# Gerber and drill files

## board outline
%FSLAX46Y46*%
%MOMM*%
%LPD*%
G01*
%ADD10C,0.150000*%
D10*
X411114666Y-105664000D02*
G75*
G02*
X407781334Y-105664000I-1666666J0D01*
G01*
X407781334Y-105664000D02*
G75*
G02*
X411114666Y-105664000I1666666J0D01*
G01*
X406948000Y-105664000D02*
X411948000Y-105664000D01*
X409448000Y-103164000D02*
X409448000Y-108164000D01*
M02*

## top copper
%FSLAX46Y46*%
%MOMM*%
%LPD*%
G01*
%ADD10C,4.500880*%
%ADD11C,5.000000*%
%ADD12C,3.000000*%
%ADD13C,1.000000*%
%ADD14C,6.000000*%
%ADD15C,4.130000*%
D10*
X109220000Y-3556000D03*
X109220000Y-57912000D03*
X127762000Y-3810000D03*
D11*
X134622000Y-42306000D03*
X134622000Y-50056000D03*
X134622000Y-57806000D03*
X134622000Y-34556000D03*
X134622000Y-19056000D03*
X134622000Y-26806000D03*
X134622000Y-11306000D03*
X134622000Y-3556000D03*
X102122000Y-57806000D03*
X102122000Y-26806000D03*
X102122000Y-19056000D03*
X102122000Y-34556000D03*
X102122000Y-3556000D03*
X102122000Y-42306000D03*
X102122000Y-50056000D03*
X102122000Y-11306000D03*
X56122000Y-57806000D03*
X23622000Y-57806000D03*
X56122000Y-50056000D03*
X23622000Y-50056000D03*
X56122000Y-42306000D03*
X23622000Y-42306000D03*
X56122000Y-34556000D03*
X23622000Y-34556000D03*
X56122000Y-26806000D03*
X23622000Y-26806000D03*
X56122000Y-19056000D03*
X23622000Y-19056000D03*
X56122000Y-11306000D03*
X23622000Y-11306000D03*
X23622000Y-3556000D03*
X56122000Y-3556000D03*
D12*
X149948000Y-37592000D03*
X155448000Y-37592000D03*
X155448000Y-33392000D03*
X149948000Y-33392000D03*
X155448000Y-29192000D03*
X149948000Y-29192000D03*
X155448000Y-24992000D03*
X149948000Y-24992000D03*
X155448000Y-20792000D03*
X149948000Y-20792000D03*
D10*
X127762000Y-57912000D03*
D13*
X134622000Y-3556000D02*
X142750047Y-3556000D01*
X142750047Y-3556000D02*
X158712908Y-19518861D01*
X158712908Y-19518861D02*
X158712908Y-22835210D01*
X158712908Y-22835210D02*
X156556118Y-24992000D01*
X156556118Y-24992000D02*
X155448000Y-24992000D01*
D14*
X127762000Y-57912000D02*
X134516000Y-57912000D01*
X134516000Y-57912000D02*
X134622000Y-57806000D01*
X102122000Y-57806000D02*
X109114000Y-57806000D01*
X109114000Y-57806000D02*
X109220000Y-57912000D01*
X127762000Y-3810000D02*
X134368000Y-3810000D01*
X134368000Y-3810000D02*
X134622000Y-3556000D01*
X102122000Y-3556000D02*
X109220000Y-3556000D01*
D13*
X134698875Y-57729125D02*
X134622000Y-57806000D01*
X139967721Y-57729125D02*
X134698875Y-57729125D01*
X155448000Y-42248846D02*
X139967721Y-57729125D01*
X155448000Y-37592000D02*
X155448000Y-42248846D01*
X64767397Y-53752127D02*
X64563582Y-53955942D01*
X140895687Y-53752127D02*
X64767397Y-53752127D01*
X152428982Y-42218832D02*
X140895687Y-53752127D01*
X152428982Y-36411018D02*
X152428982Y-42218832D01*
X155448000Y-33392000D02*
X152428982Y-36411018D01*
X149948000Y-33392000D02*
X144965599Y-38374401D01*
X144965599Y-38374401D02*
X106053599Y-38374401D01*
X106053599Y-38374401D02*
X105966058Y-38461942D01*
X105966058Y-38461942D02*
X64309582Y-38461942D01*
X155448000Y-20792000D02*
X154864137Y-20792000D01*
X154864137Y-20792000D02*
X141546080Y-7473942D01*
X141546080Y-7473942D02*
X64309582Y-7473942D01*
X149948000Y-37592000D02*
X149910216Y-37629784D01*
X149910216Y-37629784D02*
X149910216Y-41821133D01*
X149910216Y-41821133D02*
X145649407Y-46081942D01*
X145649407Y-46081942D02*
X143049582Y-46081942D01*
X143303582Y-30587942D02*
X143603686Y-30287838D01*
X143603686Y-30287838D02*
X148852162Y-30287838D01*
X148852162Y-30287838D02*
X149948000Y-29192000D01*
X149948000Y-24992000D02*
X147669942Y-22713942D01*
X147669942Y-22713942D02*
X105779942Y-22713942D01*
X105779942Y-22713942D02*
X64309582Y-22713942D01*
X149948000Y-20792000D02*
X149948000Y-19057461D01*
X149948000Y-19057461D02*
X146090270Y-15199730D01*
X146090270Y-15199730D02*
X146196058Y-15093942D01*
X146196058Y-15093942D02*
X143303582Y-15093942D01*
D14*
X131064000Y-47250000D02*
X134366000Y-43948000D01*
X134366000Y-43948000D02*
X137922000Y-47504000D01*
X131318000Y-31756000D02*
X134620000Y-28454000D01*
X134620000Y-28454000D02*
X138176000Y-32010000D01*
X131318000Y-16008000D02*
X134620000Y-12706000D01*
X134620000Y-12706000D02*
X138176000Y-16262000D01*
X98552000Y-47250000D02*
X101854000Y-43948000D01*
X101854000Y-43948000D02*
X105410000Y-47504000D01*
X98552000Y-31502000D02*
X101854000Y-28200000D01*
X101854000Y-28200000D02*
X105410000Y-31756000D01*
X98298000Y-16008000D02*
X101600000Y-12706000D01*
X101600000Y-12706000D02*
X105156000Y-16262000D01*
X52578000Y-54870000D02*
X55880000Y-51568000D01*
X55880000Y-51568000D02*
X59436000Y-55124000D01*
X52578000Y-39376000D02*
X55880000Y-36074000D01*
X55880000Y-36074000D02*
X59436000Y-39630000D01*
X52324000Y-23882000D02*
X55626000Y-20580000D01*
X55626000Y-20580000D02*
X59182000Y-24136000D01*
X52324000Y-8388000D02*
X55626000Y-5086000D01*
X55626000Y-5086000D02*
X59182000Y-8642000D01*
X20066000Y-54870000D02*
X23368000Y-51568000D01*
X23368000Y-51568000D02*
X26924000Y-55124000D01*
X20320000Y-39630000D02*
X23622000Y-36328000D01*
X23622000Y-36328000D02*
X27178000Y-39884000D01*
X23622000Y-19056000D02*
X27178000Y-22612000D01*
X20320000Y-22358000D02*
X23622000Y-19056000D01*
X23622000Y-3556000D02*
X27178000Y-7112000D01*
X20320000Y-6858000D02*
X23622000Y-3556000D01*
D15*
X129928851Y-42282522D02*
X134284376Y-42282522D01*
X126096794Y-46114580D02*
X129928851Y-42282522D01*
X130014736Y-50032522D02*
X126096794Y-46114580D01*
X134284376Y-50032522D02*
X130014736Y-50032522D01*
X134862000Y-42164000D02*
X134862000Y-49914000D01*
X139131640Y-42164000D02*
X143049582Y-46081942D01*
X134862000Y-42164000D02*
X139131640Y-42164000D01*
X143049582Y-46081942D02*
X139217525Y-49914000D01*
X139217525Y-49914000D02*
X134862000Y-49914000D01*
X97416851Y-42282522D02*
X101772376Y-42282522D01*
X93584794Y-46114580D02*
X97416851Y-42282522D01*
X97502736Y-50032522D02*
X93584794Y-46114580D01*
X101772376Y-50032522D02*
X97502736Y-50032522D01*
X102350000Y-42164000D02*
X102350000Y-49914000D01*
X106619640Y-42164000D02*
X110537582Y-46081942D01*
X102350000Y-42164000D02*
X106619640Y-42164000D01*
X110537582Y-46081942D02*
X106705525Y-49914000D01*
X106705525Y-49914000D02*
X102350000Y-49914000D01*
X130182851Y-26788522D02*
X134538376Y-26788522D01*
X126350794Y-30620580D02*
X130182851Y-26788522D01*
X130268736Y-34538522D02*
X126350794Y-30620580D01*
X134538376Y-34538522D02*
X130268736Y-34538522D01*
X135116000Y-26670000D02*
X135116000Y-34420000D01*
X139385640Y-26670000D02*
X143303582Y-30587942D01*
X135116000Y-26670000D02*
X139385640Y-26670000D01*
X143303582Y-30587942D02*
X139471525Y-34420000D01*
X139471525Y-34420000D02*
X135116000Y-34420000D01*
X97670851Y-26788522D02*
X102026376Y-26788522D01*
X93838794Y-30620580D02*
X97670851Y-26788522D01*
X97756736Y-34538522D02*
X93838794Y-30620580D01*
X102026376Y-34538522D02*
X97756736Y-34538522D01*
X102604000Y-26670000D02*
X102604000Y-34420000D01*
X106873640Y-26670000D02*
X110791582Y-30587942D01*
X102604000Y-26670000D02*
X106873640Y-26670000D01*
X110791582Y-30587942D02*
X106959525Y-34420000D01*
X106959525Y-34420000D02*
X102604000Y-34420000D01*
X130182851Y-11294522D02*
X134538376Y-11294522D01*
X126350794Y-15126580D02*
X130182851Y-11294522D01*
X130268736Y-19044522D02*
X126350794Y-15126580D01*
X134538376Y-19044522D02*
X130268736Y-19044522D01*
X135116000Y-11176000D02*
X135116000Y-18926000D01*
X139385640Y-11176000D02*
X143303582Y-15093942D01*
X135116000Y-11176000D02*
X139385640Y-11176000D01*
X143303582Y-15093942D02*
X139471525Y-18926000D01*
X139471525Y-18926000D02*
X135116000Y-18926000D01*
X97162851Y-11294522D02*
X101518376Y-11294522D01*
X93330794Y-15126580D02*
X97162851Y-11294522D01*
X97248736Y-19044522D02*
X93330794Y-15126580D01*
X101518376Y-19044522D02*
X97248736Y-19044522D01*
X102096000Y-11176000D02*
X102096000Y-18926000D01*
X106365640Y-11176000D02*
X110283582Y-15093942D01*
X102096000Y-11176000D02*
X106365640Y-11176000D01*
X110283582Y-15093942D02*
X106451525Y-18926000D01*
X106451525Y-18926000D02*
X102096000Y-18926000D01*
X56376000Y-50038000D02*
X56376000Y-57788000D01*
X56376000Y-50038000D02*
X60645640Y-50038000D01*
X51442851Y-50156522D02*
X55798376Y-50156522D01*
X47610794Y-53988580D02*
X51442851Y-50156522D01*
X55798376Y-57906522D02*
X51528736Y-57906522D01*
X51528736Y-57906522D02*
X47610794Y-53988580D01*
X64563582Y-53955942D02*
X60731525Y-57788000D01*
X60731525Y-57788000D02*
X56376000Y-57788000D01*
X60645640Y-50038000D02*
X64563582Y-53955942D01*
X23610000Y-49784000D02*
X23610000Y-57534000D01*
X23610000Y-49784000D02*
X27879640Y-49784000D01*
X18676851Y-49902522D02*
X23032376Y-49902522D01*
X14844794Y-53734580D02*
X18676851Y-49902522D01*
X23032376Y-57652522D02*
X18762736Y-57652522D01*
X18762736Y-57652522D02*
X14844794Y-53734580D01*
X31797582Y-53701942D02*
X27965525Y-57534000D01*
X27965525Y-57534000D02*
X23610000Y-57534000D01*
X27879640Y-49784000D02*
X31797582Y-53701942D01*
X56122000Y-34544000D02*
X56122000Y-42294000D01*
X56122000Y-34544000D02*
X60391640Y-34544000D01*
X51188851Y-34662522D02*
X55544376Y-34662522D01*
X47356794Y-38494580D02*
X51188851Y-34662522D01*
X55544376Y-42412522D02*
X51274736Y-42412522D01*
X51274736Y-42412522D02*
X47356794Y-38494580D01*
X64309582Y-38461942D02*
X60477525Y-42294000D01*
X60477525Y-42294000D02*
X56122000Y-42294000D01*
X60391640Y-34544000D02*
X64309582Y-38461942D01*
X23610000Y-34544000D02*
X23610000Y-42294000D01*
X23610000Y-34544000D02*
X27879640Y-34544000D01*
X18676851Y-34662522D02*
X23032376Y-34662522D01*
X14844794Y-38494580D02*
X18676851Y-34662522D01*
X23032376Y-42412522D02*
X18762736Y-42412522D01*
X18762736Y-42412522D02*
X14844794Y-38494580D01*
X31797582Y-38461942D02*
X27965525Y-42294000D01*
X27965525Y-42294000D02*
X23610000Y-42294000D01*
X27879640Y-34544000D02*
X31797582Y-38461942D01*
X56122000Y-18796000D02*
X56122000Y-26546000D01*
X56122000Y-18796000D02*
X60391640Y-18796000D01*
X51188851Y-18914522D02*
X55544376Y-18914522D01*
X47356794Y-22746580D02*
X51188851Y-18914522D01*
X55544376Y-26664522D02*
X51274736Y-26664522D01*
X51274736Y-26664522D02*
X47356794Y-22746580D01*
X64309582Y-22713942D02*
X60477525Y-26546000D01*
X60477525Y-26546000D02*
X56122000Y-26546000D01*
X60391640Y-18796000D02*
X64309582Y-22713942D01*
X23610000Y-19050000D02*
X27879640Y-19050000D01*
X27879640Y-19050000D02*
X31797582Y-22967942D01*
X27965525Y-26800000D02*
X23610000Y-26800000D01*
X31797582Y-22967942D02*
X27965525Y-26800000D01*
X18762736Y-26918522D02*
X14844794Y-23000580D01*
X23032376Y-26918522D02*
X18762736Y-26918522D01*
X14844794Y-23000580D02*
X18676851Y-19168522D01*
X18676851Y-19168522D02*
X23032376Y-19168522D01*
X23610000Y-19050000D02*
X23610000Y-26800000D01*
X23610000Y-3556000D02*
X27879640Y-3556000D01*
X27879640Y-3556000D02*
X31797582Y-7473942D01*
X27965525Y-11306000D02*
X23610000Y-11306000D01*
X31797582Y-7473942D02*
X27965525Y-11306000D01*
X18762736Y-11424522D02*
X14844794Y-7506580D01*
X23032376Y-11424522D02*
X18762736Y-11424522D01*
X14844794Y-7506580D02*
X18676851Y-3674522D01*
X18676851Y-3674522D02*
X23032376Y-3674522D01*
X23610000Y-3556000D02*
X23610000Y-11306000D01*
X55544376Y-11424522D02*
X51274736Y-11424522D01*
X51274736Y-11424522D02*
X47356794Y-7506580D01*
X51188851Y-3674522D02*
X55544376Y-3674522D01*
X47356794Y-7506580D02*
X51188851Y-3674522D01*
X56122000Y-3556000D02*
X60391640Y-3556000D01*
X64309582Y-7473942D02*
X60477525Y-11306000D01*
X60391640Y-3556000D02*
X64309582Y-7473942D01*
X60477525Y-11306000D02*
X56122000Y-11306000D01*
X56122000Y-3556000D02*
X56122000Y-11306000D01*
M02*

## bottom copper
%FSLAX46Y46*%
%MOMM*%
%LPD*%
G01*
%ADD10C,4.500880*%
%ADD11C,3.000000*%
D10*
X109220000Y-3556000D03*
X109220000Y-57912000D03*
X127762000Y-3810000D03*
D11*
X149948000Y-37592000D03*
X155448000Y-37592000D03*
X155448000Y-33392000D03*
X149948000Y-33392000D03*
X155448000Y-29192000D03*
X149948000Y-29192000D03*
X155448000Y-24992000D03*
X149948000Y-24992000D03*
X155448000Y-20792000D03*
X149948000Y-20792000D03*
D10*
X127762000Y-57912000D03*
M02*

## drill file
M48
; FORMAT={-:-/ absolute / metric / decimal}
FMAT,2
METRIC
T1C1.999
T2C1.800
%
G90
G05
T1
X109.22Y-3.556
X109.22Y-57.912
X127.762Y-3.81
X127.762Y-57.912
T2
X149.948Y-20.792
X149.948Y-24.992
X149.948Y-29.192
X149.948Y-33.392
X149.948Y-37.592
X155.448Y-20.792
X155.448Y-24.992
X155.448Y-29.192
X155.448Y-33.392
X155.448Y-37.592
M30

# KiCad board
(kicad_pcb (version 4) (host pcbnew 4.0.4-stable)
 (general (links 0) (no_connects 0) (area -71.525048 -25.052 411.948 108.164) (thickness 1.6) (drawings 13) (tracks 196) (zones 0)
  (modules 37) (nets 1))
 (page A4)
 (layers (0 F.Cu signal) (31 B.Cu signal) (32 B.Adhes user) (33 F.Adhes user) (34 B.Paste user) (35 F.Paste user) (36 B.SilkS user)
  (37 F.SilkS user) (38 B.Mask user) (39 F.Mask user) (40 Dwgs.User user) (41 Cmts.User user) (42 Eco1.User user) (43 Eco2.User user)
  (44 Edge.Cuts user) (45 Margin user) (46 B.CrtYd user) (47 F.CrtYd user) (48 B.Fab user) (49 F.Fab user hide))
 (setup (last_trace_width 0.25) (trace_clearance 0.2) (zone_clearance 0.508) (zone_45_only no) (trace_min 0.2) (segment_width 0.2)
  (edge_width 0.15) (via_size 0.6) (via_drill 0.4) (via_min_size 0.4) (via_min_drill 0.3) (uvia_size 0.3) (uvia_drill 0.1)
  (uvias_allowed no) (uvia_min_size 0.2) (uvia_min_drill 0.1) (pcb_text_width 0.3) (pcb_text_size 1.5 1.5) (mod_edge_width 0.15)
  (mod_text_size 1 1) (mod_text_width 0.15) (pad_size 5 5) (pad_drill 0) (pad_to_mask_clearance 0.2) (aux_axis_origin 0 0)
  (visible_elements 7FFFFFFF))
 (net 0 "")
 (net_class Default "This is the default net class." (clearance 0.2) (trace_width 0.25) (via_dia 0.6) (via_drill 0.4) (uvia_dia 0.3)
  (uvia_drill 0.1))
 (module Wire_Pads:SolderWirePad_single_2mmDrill (layer F.Cu) (at 109.22 3.556)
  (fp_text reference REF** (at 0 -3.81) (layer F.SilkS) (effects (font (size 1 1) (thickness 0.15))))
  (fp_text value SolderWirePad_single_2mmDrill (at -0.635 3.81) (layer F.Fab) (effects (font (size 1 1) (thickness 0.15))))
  (pad 1 thru_hole circle (at 0 0) (size 4.50088 4.50088) (drill 1.99898) (layers *.Cu *.Mask)))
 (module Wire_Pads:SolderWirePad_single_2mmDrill (layer F.Cu) (at 109.22 57.912)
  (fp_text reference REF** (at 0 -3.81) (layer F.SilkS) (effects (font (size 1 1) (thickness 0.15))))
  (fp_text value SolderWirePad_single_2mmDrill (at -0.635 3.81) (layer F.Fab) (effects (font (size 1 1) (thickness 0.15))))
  (pad 1 thru_hole circle (at 0 0) (size 4.50088 4.50088) (drill 1.99898) (layers *.Cu *.Mask)))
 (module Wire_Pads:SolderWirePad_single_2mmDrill (layer F.Cu) (at 127.762 3.81)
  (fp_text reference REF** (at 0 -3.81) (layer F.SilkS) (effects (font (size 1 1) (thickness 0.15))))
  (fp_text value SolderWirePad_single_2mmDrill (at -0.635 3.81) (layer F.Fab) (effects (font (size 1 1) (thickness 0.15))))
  (pad 1 thru_hole circle (at 0 0) (size 4.50088 4.50088) (drill 1.99898) (layers *.Cu *.Mask)))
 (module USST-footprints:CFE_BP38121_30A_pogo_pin (layer F.Cu) (at 174.5 53.736)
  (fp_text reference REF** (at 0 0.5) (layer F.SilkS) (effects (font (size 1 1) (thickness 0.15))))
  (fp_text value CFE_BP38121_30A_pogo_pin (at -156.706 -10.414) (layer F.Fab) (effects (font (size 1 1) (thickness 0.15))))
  (pad 6 smd circle (at -39.878 -11.43) (size 5 5) (layers F.Cu F.Paste F.Mask)))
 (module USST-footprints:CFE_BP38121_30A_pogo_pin (layer F.Cu) (at 174.5 61.486)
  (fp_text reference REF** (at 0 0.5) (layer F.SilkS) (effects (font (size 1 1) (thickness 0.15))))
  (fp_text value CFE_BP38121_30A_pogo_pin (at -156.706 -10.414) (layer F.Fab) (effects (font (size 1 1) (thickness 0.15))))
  (pad 7 smd circle (at -39.878 -11.43) (size 5 5) (layers F.Cu F.Paste F.Mask)))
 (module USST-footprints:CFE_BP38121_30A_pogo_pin (layer F.Cu) (at 174.5 69.236)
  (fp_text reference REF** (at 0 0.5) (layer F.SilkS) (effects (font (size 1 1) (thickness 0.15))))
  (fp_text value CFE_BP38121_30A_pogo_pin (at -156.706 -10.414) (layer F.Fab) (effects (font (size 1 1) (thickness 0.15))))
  (pad 8 smd circle (at -39.878 -11.43) (size 5 5) (layers F.Cu F.Paste F.Mask)))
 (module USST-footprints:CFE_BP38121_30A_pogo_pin (layer F.Cu) (at 174.5 45.986)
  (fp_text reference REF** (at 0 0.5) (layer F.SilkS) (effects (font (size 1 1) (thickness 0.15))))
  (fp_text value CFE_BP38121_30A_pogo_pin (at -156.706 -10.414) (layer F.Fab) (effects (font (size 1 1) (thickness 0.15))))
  (pad 5 smd circle (at -39.878 -11.43) (size 5 5) (layers F.Cu F.Paste F.Mask)))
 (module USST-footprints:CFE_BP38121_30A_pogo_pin (layer F.Cu) (at 174.5 30.486)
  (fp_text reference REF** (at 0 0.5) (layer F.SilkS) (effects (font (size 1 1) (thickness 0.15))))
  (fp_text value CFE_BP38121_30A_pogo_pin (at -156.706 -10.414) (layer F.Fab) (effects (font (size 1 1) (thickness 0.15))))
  (pad 3 smd circle (at -39.878 -11.43) (size 5 5) (layers F.Cu F.Paste F.Mask)))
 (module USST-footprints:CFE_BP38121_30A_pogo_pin (layer F.Cu) (at 174.5 38.236)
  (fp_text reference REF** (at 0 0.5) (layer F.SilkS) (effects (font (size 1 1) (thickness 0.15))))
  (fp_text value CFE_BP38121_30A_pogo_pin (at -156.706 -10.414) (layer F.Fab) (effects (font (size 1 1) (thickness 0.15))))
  (pad 4 smd circle (at -39.878 -11.43) (size 5 5) (layers F.Cu F.Paste F.Mask)))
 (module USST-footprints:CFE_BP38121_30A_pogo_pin (layer F.Cu) (at 174.5 22.736)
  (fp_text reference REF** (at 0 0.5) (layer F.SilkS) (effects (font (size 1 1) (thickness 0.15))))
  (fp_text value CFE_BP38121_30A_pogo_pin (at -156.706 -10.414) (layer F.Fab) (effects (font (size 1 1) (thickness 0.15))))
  (pad 2 smd circle (at -39.878 -11.43) (size 5 5) (layers F.Cu F.Paste F.Mask)))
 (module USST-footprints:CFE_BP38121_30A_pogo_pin (layer F.Cu) (at 174.5 14.986)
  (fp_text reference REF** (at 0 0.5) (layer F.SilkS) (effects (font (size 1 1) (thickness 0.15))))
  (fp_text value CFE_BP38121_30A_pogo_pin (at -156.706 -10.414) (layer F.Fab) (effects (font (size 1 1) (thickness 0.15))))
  (pad 1 smd circle (at -39.878 -11.43) (size 5 5) (layers F.Cu F.Paste F.Mask)))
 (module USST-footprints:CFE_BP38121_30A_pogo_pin (layer F.Cu) (at 142 69.236)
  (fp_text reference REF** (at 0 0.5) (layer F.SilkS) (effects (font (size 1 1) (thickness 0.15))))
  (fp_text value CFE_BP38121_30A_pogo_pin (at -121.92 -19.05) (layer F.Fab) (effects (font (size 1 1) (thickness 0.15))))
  (pad 8 smd circle (at -39.878 -11.43) (size 5 5) (layers F.Cu F.Paste F.Mask)))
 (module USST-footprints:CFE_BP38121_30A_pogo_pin (layer F.Cu) (at 142 38.236)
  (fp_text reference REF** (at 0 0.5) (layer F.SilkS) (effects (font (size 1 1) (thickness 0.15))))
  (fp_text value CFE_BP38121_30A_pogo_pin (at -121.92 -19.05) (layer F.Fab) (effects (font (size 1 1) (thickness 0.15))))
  (pad 4 smd circle (at -39.878 -11.43) (size 5 5) (layers F.Cu F.Paste F.Mask)))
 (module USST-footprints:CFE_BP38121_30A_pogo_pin (layer F.Cu) (at 142 30.486)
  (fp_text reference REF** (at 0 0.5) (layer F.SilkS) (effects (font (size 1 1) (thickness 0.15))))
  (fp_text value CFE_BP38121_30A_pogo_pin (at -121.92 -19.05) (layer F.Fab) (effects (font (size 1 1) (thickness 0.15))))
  (pad 3 smd circle (at -39.878 -11.43) (size 5 5) (layers F.Cu F.Paste F.Mask)))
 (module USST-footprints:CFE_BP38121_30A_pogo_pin (layer F.Cu) (at 142 45.986)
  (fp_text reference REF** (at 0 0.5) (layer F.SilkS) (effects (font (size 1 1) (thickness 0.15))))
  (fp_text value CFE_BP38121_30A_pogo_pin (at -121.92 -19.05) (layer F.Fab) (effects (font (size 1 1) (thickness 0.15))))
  (pad 5 smd circle (at -39.878 -11.43) (size 5 5) (layers F.Cu F.Paste F.Mask)))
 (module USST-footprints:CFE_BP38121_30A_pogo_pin (layer F.Cu) (at 142 14.986)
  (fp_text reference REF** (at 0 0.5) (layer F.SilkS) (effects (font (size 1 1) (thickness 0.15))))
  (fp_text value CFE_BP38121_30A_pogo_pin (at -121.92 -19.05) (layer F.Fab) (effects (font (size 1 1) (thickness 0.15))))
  (pad 1 smd circle (at -39.878 -11.43) (size 5 5) (layers F.Cu F.Paste F.Mask)))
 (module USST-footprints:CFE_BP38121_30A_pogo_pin (layer F.Cu) (at 142 53.736)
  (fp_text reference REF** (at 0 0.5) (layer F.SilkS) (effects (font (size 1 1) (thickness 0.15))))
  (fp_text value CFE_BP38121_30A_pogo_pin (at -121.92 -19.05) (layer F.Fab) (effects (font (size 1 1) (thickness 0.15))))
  (pad 6 smd circle (at -39.878 -11.43) (size 5 5) (layers F.Cu F.Paste F.Mask)))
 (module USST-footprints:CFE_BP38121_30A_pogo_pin (layer F.Cu) (at 142 61.486)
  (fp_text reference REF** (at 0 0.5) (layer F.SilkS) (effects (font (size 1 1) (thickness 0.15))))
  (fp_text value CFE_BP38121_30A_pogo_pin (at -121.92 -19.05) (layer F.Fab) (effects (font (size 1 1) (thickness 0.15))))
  (pad 7 smd circle (at -39.878 -11.43) (size 5 5) (layers F.Cu F.Paste F.Mask)))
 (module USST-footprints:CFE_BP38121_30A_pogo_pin (layer F.Cu) (at 142 22.736)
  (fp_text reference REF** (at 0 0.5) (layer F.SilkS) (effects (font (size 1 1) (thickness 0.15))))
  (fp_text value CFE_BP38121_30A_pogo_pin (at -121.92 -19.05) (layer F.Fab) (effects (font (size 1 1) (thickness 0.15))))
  (pad 2 smd circle (at -39.878 -11.43) (size 5 5) (layers F.Cu F.Paste F.Mask)))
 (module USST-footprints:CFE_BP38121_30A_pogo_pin (layer F.Cu) (at 96 69.236)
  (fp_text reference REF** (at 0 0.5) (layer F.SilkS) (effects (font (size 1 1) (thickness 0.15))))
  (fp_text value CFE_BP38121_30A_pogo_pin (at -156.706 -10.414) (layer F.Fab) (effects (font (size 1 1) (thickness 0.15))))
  (pad 8 smd circle (at -39.878 -11.43) (size 5 5) (layers F.Cu F.Paste F.Mask)))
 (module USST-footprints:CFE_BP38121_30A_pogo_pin (layer F.Cu) (at 63.5 69.236)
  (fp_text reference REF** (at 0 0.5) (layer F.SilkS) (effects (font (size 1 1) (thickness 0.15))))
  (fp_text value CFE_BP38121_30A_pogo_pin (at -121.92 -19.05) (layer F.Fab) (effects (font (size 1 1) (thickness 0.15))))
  (pad 8 smd circle (at -39.878 -11.43) (size 5 5) (layers F.Cu F.Paste F.Mask)))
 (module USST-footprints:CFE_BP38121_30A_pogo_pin (layer F.Cu) (at 96 61.486)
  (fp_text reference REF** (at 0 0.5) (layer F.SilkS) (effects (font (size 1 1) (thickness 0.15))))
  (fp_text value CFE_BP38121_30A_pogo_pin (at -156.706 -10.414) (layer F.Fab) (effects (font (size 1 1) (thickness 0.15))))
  (pad 7 smd circle (at -39.878 -11.43) (size 5 5) (layers F.Cu F.Paste F.Mask)))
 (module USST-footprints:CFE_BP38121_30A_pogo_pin (layer F.Cu) (at 63.5 61.486)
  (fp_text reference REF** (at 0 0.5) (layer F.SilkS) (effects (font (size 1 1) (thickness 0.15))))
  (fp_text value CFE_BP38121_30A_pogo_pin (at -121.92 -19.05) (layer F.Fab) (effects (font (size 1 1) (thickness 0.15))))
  (pad 7 smd circle (at -39.878 -11.43) (size 5 5) (layers F.Cu F.Paste F.Mask)))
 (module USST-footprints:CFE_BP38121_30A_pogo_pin (layer F.Cu) (at 96 53.736)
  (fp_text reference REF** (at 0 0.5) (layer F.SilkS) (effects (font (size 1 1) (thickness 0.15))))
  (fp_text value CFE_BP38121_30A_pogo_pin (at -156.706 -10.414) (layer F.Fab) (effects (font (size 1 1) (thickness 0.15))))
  (pad 6 smd circle (at -39.878 -11.43) (size 5 5) (layers F.Cu F.Paste F.Mask)))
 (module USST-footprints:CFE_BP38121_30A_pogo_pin (layer F.Cu) (at 63.5 53.736)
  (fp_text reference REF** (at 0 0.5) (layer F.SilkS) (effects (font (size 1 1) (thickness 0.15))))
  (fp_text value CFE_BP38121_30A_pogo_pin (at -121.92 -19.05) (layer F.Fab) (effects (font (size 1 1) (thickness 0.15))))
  (pad 6 smd circle (at -39.878 -11.43) (size 5 5) (layers F.Cu F.Paste F.Mask)))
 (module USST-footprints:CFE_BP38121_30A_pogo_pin (layer F.Cu) (at 96 45.986)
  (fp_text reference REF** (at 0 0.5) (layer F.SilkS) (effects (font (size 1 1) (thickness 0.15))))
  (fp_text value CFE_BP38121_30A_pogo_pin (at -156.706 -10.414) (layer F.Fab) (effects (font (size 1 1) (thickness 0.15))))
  (pad 5 smd circle (at -39.878 -11.43) (size 5 5) (layers F.Cu F.Paste F.Mask)))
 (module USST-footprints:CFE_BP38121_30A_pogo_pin (layer F.Cu) (at 63.5 45.986)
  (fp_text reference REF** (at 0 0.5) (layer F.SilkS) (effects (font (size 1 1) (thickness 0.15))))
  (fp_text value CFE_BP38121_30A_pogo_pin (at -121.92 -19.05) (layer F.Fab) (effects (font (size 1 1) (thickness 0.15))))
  (pad 5 smd circle (at -39.878 -11.43) (size 5 5) (layers F.Cu F.Paste F.Mask)))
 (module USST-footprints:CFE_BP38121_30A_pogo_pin (layer F.Cu) (at 96 38.236)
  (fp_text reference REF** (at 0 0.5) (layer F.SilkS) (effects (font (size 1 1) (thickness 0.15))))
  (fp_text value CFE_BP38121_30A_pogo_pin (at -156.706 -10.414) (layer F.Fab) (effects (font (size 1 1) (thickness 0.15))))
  (pad 4 smd circle (at -39.878 -11.43) (size 5 5) (layers F.Cu F.Paste F.Mask)))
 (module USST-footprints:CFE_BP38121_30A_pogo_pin (layer F.Cu) (at 63.5 38.236)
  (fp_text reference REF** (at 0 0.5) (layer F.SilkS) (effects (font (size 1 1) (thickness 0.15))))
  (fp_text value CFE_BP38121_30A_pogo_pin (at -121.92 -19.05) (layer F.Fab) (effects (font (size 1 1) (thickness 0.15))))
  (pad 4 smd circle (at -39.878 -11.43) (size 5 5) (layers F.Cu F.Paste F.Mask)))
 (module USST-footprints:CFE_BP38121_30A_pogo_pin (layer F.Cu) (at 96 30.486)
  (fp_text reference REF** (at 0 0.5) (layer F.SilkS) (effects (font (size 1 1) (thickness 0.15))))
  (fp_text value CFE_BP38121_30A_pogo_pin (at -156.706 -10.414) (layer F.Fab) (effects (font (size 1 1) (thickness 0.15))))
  (pad 3 smd circle (at -39.878 -11.43) (size 5 5) (layers F.Cu F.Paste F.Mask)))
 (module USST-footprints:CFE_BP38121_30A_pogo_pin (layer F.Cu) (at 63.5 30.486)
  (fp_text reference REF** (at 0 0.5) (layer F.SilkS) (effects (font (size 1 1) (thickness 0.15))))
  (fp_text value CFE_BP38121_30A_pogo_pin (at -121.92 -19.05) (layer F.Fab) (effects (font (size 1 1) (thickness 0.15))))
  (pad 3 smd circle (at -39.878 -11.43) (size 5 5) (layers F.Cu F.Paste F.Mask)))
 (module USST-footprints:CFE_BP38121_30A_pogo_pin (layer F.Cu) (at 96 22.736)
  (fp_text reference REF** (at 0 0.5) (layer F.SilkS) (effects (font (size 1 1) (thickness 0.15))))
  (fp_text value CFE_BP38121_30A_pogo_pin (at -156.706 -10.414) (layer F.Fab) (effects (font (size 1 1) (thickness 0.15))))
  (pad 2 smd circle (at -39.878 -11.43) (size 5 5) (layers F.Cu F.Paste F.Mask)))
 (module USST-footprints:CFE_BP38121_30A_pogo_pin (layer F.Cu) (at 63.5 22.736)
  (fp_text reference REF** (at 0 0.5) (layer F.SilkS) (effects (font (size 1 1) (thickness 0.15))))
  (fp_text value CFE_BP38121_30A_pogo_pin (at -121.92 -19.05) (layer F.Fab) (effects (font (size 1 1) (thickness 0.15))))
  (pad 2 smd circle (at -39.878 -11.43) (size 5 5) (layers F.Cu F.Paste F.Mask)))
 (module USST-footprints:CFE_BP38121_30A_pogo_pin (layer F.Cu) (at 63.5 14.986)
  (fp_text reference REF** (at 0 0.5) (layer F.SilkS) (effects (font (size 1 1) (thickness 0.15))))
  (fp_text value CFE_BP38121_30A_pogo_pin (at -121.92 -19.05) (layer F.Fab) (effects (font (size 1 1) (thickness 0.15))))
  (pad 1 smd circle (at -39.878 -11.43) (size 5 5) (layers F.Cu F.Paste F.Mask)))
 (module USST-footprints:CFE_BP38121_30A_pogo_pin (layer F.Cu) (at 96 14.986)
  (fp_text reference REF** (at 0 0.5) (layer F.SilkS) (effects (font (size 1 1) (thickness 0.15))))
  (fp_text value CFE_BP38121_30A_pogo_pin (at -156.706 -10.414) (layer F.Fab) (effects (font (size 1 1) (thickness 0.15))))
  (pad 1 smd circle (at -39.878 -11.43) (size 5 5) (layers F.Cu F.Paste F.Mask)))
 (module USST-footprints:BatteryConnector (layer F.Cu) (at 149.948 37.592)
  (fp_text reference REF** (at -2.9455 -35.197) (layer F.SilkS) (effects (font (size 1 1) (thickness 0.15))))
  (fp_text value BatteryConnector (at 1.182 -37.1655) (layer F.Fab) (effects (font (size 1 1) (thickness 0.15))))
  (pad "" np_thru_hole circle (at 0 0) (size 3 3) (drill 1.8) (layers *.Cu))
  (pad "" np_thru_hole circle (at 5.5 0) (size 3 3) (drill 1.8) (layers *.Cu))
  (pad "" np_thru_hole circle (at 5.5 -4.2) (size 3 3) (drill 1.8) (layers *.Cu))
  (pad "" np_thru_hole circle (at 0 -4.2) (size 3 3) (drill 1.8) (layers *.Cu))
  (pad "" np_thru_hole circle (at 5.5 -8.4) (size 3 3) (drill 1.8) (layers *.Cu))
  (pad "" np_thru_hole circle (at 0 -8.4) (size 3 3) (drill 1.8) (layers *.Cu))
  (pad "" np_thru_hole circle (at 5.5 -12.6) (size 3 3) (drill 1.8) (layers *.Cu))
  (pad "" np_thru_hole circle (at 0 -12.6) (size 3 3) (drill 1.8) (layers *.Cu))
  (pad "" np_thru_hole circle (at 5.5 -16.8) (size 3 3) (drill 1.8) (layers *.Cu))
  (pad "" np_thru_hole circle (at 0 -16.8) (size 3 3) (drill 1.8) (layers *.Cu)))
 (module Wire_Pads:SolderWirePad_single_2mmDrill (layer F.Cu) (at 127.762 57.912)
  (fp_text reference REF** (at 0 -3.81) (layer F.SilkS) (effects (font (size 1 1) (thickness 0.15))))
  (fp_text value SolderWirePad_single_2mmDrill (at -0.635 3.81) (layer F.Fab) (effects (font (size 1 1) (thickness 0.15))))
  (pad 1 thru_hole circle (at 0 0) (size 4.50088 4.50088) (drill 1.99898) (layers *.Cu *.Mask)))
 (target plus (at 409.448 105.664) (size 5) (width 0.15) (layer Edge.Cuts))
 (segment (start 134.622 3.556) (end 142.750047 3.556) (width 1) (layer F.Cu) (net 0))
 (segment (start 142.750047 3.556) (end 158.712908 19.518861) (width 1) (layer F.Cu) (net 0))
 (segment (start 158.712908 19.518861) (end 158.712908 22.83521) (width 1) (layer F.Cu) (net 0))
 (segment (start 158.712908 22.83521) (end 156.556118 24.992) (width 1) (layer F.Cu) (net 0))
 (segment (start 156.556118 24.992) (end 155.448 24.992) (width 1) (layer F.Cu) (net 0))
 (segment (start 127.762 57.912) (end 134.516 57.912) (width 6) (layer F.Cu) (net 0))
 (segment (start 134.516 57.912) (end 134.622 57.806) (width 6) (layer F.Cu) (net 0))
 (segment (start 102.122 57.806) (end 109.114 57.806) (width 6) (layer F.Cu) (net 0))
 (segment (start 109.114 57.806) (end 109.22 57.912) (width 6) (layer F.Cu) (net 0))
 (segment (start 127.762 3.81) (end 134.368 3.81) (width 6) (layer F.Cu) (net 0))
 (segment (start 134.368 3.81) (end 134.622 3.556) (width 6) (layer F.Cu) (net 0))
 (segment (start 102.122 3.556) (end 109.22 3.556) (width 6) (layer F.Cu) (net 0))
 (segment (start 134.698875 57.729125) (end 134.622 57.806) (width 1) (layer F.Cu) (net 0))
 (segment (start 139.967721 57.729125) (end 134.698875 57.729125) (width 1) (layer F.Cu) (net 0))
 (segment (start 155.448 42.248846) (end 139.967721 57.729125) (width 1) (layer F.Cu) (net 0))
 (segment (start 155.448 37.592) (end 155.448 42.248846) (width 1) (layer F.Cu) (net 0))
 (segment (start 64.767397 53.752127) (end 64.563582 53.955942) (width 1) (layer F.Cu) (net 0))
 (segment (start 140.895687 53.752127) (end 64.767397 53.752127) (width 1) (layer F.Cu) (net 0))
 (segment (start 152.428982 42.218832) (end 140.895687 53.752127) (width 1) (layer F.Cu) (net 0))
 (segment (start 152.428982 36.411018) (end 152.428982 42.218832) (width 1) (layer F.Cu) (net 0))
 (segment (start 155.448 33.392) (end 152.428982 36.411018) (width 1) (layer F.Cu) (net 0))
 (segment (start 149.948 33.392) (end 144.965599 38.374401) (width 1) (layer F.Cu) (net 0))
 (segment (start 144.965599 38.374401) (end 106.053599 38.374401) (width 1) (layer F.Cu) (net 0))
 (segment (start 106.053599 38.374401) (end 105.966058 38.461942) (width 1) (layer F.Cu) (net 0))
 (segment (start 105.966058 38.461942) (end 64.309582 38.461942) (width 1) (layer F.Cu) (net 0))
 (segment (start 155.448 20.792) (end 154.864137 20.792) (width 1) (layer F.Cu) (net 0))
 (segment (start 154.864137 20.792) (end 141.54608 7.473942) (width 1) (layer F.Cu) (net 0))
 (segment (start 141.54608 7.473942) (end 64.309582 7.473942) (width 1) (layer F.Cu) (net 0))
 (segment (start 149.948 37.592) (end 149.910216 37.629784) (width 1) (layer F.Cu) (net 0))
 (segment (start 149.910216 37.629784) (end 149.910216 41.821133) (width 1) (layer F.Cu) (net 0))
 (segment (start 149.910216 41.821133) (end 145.649407 46.081942) (width 1) (layer F.Cu) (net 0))
 (segment (start 145.649407 46.081942) (end 143.049582 46.081942) (width 1) (layer F.Cu) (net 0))
 (segment (start 143.303582 30.587942) (end 143.603686 30.287838) (width 1) (layer F.Cu) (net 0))
 (segment (start 143.603686 30.287838) (end 148.852162 30.287838) (width 1) (layer F.Cu) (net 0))
 (segment (start 148.852162 30.287838) (end 149.948 29.192) (width 1) (layer F.Cu) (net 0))
 (segment (start 149.948 24.992) (end 147.669942 22.713942) (width 1) (layer F.Cu) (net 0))
 (segment (start 147.669942 22.713942) (end 105.779942 22.713942) (width 1) (layer F.Cu) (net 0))
 (segment (start 105.779942 22.713942) (end 64.309582 22.713942) (width 1) (layer F.Cu) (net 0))
 (segment (start 149.948 20.792) (end 149.948 19.057461) (width 1) (layer F.Cu) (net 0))
 (segment (start 149.948 19.057461) (end 146.09027 15.19973) (width 1) (layer F.Cu) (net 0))
 (segment (start 146.09027 15.19973) (end 146.196058 15.093942) (width 1) (layer F.Cu) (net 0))
 (segment (start 146.196058 15.093942) (end 143.303582 15.093942) (width 1) (layer F.Cu) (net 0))
 (segment (start 131.064 47.25) (end 134.366 43.948) (width 6) (layer F.Cu) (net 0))
 (segment (start 134.366 43.948) (end 137.922 47.504) (width 6) (layer F.Cu) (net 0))
 (segment (start 131.318 31.756) (end 134.62 28.454) (width 6) (layer F.Cu) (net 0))
 (segment (start 134.62 28.454) (end 138.176 32.01) (width 6) (layer F.Cu) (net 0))
 (segment (start 131.318 16.008) (end 134.62 12.706) (width 6) (layer F.Cu) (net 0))
 (segment (start 134.62 12.706) (end 138.176 16.262) (width 6) (layer F.Cu) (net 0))
 (segment (start 98.552 47.25) (end 101.854 43.948) (width 6) (layer F.Cu) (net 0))
 (segment (start 101.854 43.948) (end 105.41 47.504) (width 6) (layer F.Cu) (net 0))
 (segment (start 98.552 31.502) (end 101.854 28.2) (width 6) (layer F.Cu) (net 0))
 (segment (start 101.854 28.2) (end 105.41 31.756) (width 6) (layer F.Cu) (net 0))
 (segment (start 98.298 16.008) (end 101.6 12.706) (width 6) (layer F.Cu) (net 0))
 (segment (start 101.6 12.706) (end 105.156 16.262) (width 6) (layer F.Cu) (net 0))
 (segment (start 52.578 54.87) (end 55.88 51.568) (width 6) (layer F.Cu) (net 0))
 (segment (start 55.88 51.568) (end 59.436 55.124) (width 6) (layer F.Cu) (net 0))
 (segment (start 52.578 39.376) (end 55.88 36.074) (width 6) (layer F.Cu) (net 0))
 (segment (start 55.88 36.074) (end 59.436 39.63) (width 6) (layer F.Cu) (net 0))
 (segment (start 52.324 23.882) (end 55.626 20.58) (width 6) (layer F.Cu) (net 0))
 (segment (start 55.626 20.58) (end 59.182 24.136) (width 6) (layer F.Cu) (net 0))
 (segment (start 52.324 8.388) (end 55.626 5.086) (width 6) (layer F.Cu) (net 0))
 (segment (start 55.626 5.086) (end 59.182 8.642) (width 6) (layer F.Cu) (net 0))
 (segment (start 20.066 54.87) (end 23.368 51.568) (width 6) (layer F.Cu) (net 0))
 (segment (start 23.368 51.568) (end 26.924 55.124) (width 6) (layer F.Cu) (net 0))
 (segment (start 20.32 39.63) (end 23.622 36.328) (width 6) (layer F.Cu) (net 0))
 (segment (start 23.622 36.328) (end 27.178 39.884) (width 6) (layer F.Cu) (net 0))
 (segment (start 23.622 19.056) (end 27.178 22.612) (width 6) (layer F.Cu) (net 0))
 (segment (start 20.32 22.358) (end 23.622 19.056) (width 6) (layer F.Cu) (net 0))
 (segment (start 23.622 3.556) (end 27.178 7.112) (width 6) (layer F.Cu) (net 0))
 (segment (start 20.32 6.858) (end 23.622 3.556) (width 6) (layer F.Cu) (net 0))
 (segment (start 129.928851 42.282522) (end 134.284376 42.282522) (width 4.13) (layer F.Cu) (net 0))
 (segment (start 126.096794 46.11458) (end 129.928851 42.282522) (width 4.13) (layer F.Cu) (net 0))
 (segment (start 130.014736 50.032522) (end 126.096794 46.11458) (width 4.13) (layer F.Cu) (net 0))
 (segment (start 134.284376 50.032522) (end 130.014736 50.032522) (width 4.13) (layer F.Cu) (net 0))
 (segment (start 134.862 42.164) (end 134.862 49.914) (width 4.13) (layer F.Cu) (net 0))
 (segment (start 139.13164 42.164) (end 143.049582 46.081942) (width 4.13) (layer F.Cu) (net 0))
 (segment (start 134.862 42.164) (end 139.13164 42.164) (width 4.13) (layer F.Cu) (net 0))
 (segment (start 143.049582 46.081942) (end 139.217525 49.914) (width 4.13) (layer F.Cu) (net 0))
 (segment (start 139.217525 49.914) (end 134.862 49.914) (width 4.13) (layer F.Cu) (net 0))
 (segment (start 97.416851 42.282522) (end 101.772376 42.282522) (width 4.13) (layer F.Cu) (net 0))
 (segment (start 93.584794 46.11458) (end 97.416851 42.282522) (width 4.13) (layer F.Cu) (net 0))
 (segment (start 97.502736 50.032522) (end 93.584794 46.11458) (width 4.13) (layer F.Cu) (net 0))
 (segment (start 101.772376 50.032522) (end 97.502736 50.032522) (width 4.13) (layer F.Cu) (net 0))
 (segment (start 102.35 42.164) (end 102.35 49.914) (width 4.13) (layer F.Cu) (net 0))
 (segment (start 106.61964 42.164) (end 110.537582 46.081942) (width 4.13) (layer F.Cu) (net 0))
 (segment (start 102.35 42.164) (end 106.61964 42.164) (width 4.13) (layer F.Cu) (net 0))
 (segment (start 110.537582 46.081942) (end 106.705525 49.914) (width 4.13) (layer F.Cu) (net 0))
 (segment (start 106.705525 49.914) (end 102.35 49.914) (width 4.13) (layer F.Cu) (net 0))
 (segment (start 130.182851 26.788522) (end 134.538376 26.788522) (width 4.13) (layer F.Cu) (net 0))
 (segment (start 126.350794 30.62058) (end 130.182851 26.788522) (width 4.13) (layer F.Cu) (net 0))
 (segment (start 130.268736 34.538522) (end 126.350794 30.62058) (width 4.13) (layer F.Cu) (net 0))
 (segment (start 134.538376 34.538522) (end 130.268736 34.538522) (width 4.13) (layer F.Cu) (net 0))
 (segment (start 135.116 26.67) (end 135.116 34.42) (width 4.13) (layer F.Cu) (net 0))
 (segment (start 139.38564 26.67) (end 143.303582 30.587942) (width 4.13) (layer F.Cu) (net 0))
 (segment (start 135.116 26.67) (end 139.38564 26.67) (width 4.13) (layer F.Cu) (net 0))
 (segment (start 143.303582 30.587942) (end 139.471525 34.42) (width 4.13) (layer F.Cu) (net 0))
 (segment (start 139.471525 34.42) (end 135.116 34.42) (width 4.13) (layer F.Cu) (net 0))
 (segment (start 97.670851 26.788522) (end 102.026376 26.788522) (width 4.13) (layer F.Cu) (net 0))
 (segment (start 93.838794 30.62058) (end 97.670851 26.788522) (width 4.13) (layer F.Cu) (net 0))
 (segment (start 97.756736 34.538522) (end 93.838794 30.62058) (width 4.13) (layer F.Cu) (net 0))
 (segment (start 102.026376 34.538522) (end 97.756736 34.538522) (width 4.13) (layer F.Cu) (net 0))
 (segment (start 102.604 26.67) (end 102.604 34.42) (width 4.13) (layer F.Cu) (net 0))
 (segment (start 106.87364 26.67) (end 110.791582 30.587942) (width 4.13) (layer F.Cu) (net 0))
 (segment (start 102.604 26.67) (end 106.87364 26.67) (width 4.13) (layer F.Cu) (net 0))
 (segment (start 110.791582 30.587942) (end 106.959525 34.42) (width 4.13) (layer F.Cu) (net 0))
 (segment (start 106.959525 34.42) (end 102.604 34.42) (width 4.13) (layer F.Cu) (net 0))
 (segment (start 130.182851 11.294522) (end 134.538376 11.294522) (width 4.13) (layer F.Cu) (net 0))
 (segment (start 126.350794 15.12658) (end 130.182851 11.294522) (width 4.13) (layer F.Cu) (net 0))
 (segment (start 130.268736 19.044522) (end 126.350794 15.12658) (width 4.13) (layer F.Cu) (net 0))
 (segment (start 134.538376 19.044522) (end 130.268736 19.044522) (width 4.13) (layer F.Cu) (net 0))
 (segment (start 135.116 11.176) (end 135.116 18.926) (width 4.13) (layer F.Cu) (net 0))
 (segment (start 139.38564 11.176) (end 143.303582 15.093942) (width 4.13) (layer F.Cu) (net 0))
 (segment (start 135.116 11.176) (end 139.38564 11.176) (width 4.13) (layer F.Cu) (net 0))
 (segment (start 143.303582 15.093942) (end 139.471525 18.926) (width 4.13) (layer F.Cu) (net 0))
 (segment (start 139.471525 18.926) (end 135.116 18.926) (width 4.13) (layer F.Cu) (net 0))
 (segment (start 97.162851 11.294522) (end 101.518376 11.294522) (width 4.13) (layer F.Cu) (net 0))
 (segment (start 93.330794 15.12658) (end 97.162851 11.294522) (width 4.13) (layer F.Cu) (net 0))
 (segment (start 97.248736 19.044522) (end 93.330794 15.12658) (width 4.13) (layer F.Cu) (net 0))
 (segment (start 101.518376 19.044522) (end 97.248736 19.044522) (width 4.13) (layer F.Cu) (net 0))
 (segment (start 102.096 11.176) (end 102.096 18.926) (width 4.13) (layer F.Cu) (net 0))
 (segment (start 106.36564 11.176) (end 110.283582 15.093942) (width 4.13) (layer F.Cu) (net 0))
 (segment (start 102.096 11.176) (end 106.36564 11.176) (width 4.13) (layer F.Cu) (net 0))
 (segment (start 110.283582 15.093942) (end 106.451525 18.926) (width 4.13) (layer F.Cu) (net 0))
 (segment (start 106.451525 18.926) (end 102.096 18.926) (width 4.13) (layer F.Cu) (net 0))
 (segment (start 56.376 50.038) (end 56.376 57.788) (width 4.13) (layer F.Cu) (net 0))
 (segment (start 56.376 50.038) (end 60.64564 50.038) (width 4.13) (layer F.Cu) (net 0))
 (segment (start 51.442851 50.156522) (end 55.798376 50.156522) (width 4.13) (layer F.Cu) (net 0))
 (segment (start 47.610794 53.98858) (end 51.442851 50.156522) (width 4.13) (layer F.Cu) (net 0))
 (segment (start 55.798376 57.906522) (end 51.528736 57.906522) (width 4.13) (layer F.Cu) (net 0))
 (segment (start 51.528736 57.906522) (end 47.610794 53.98858) (width 4.13) (layer F.Cu) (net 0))
 (segment (start 64.563582 53.955942) (end 60.731525 57.788) (width 4.13) (layer F.Cu) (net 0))
 (segment (start 60.731525 57.788) (end 56.376 57.788) (width 4.13) (layer F.Cu) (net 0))
 (segment (start 60.64564 50.038) (end 64.563582 53.955942) (width 4.13) (layer F.Cu) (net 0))
 (segment (start 23.61 49.784) (end 23.61 57.534) (width 4.13) (layer F.Cu) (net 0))
 (segment (start 23.61 49.784) (end 27.87964 49.784) (width 4.13) (layer F.Cu) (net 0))
 (segment (start 18.676851 49.902522) (end 23.032376 49.902522) (width 4.13) (layer F.Cu) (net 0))
 (segment (start 14.844794 53.73458) (end 18.676851 49.902522) (width 4.13) (layer F.Cu) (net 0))
 (segment (start 23.032376 57.652522) (end 18.762736 57.652522) (width 4.13) (layer F.Cu) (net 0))
 (segment (start 18.762736 57.652522) (end 14.844794 53.73458) (width 4.13) (layer F.Cu) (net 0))
 (segment (start 31.797582 53.701942) (end 27.965525 57.534) (width 4.13) (layer F.Cu) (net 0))
 (segment (start 27.965525 57.534) (end 23.61 57.534) (width 4.13) (layer F.Cu) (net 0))
 (segment (start 27.87964 49.784) (end 31.797582 53.701942) (width 4.13) (layer F.Cu) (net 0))
 (segment (start 56.122 34.544) (end 56.122 42.294) (width 4.13) (layer F.Cu) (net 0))
 (segment (start 56.122 34.544) (end 60.39164 34.544) (width 4.13) (layer F.Cu) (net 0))
 (segment (start 51.188851 34.662522) (end 55.544376 34.662522) (width 4.13) (layer F.Cu) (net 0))
 (segment (start 47.356794 38.49458) (end 51.188851 34.662522) (width 4.13) (layer F.Cu) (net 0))
 (segment (start 55.544376 42.412522) (end 51.274736 42.412522) (width 4.13) (layer F.Cu) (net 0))
 (segment (start 51.274736 42.412522) (end 47.356794 38.49458) (width 4.13) (layer F.Cu) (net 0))
 (segment (start 64.309582 38.461942) (end 60.477525 42.294) (width 4.13) (layer F.Cu) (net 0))
 (segment (start 60.477525 42.294) (end 56.122 42.294) (width 4.13) (layer F.Cu) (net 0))
 (segment (start 60.39164 34.544) (end 64.309582 38.461942) (width 4.13) (layer F.Cu) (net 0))
 (segment (start 23.61 34.544) (end 23.61 42.294) (width 4.13) (layer F.Cu) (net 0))
 (segment (start 23.61 34.544) (end 27.87964 34.544) (width 4.13) (layer F.Cu) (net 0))
 (segment (start 18.676851 34.662522) (end 23.032376 34.662522) (width 4.13) (layer F.Cu) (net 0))
 (segment (start 14.844794 38.49458) (end 18.676851 34.662522) (width 4.13) (layer F.Cu) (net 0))
 (segment (start 23.032376 42.412522) (end 18.762736 42.412522) (width 4.13) (layer F.Cu) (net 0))
 (segment (start 18.762736 42.412522) (end 14.844794 38.49458) (width 4.13) (layer F.Cu) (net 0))
 (segment (start 31.797582 38.461942) (end 27.965525 42.294) (width 4.13) (layer F.Cu) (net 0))
 (segment (start 27.965525 42.294) (end 23.61 42.294) (width 4.13) (layer F.Cu) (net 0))
 (segment (start 27.87964 34.544) (end 31.797582 38.461942) (width 4.13) (layer F.Cu) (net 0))
 (segment (start 56.122 18.796) (end 56.122 26.546) (width 4.13) (layer F.Cu) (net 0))
 (segment (start 56.122 18.796) (end 60.39164 18.796) (width 4.13) (layer F.Cu) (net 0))
 (segment (start 51.188851 18.914522) (end 55.544376 18.914522) (width 4.13) (layer F.Cu) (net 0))
 (segment (start 47.356794 22.74658) (end 51.188851 18.914522) (width 4.13) (layer F.Cu) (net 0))
 (segment (start 55.544376 26.664522) (end 51.274736 26.664522) (width 4.13) (layer F.Cu) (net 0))
 (segment (start 51.274736 26.664522) (end 47.356794 22.74658) (width 4.13) (layer F.Cu) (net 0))
 (segment (start 64.309582 22.713942) (end 60.477525 26.546) (width 4.13) (layer F.Cu) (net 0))
 (segment (start 60.477525 26.546) (end 56.122 26.546) (width 4.13) (layer F.Cu) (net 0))
 (segment (start 60.39164 18.796) (end 64.309582 22.713942) (width 4.13) (layer F.Cu) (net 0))
 (segment (start 23.61 19.05) (end 27.87964 19.05) (width 4.13) (layer F.Cu) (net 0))
 (segment (start 27.87964 19.05) (end 31.797582 22.967942) (width 4.13) (layer F.Cu) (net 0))
 (segment (start 27.965525 26.8) (end 23.61 26.8) (width 4.13) (layer F.Cu) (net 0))
 (segment (start 31.797582 22.967942) (end 27.965525 26.8) (width 4.13) (layer F.Cu) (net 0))
 (segment (start 18.762736 26.918522) (end 14.844794 23.00058) (width 4.13) (layer F.Cu) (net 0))
 (segment (start 23.032376 26.918522) (end 18.762736 26.918522) (width 4.13) (layer F.Cu) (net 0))
 (segment (start 14.844794 23.00058) (end 18.676851 19.168522) (width 4.13) (layer F.Cu) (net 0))
 (segment (start 18.676851 19.168522) (end 23.032376 19.168522) (width 4.13) (layer F.Cu) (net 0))
 (segment (start 23.61 19.05) (end 23.61 26.8) (width 4.13) (layer F.Cu) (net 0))
 (segment (start 23.61 3.556) (end 27.87964 3.556) (width 4.13) (layer F.Cu) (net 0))
 (segment (start 27.87964 3.556) (end 31.797582 7.473942) (width 4.13) (layer F.Cu) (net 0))
 (segment (start 27.965525 11.306) (end 23.61 11.306) (width 4.13) (layer F.Cu) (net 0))
 (segment (start 31.797582 7.473942) (end 27.965525 11.306) (width 4.13) (layer F.Cu) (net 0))
 (segment (start 18.762736 11.424522) (end 14.844794 7.50658) (width 4.13) (layer F.Cu) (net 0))
 (segment (start 23.032376 11.424522) (end 18.762736 11.424522) (width 4.13) (layer F.Cu) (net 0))
 (segment (start 14.844794 7.50658) (end 18.676851 3.674522) (width 4.13) (layer F.Cu) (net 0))
 (segment (start 18.676851 3.674522) (end 23.032376 3.674522) (width 4.13) (layer F.Cu) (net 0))
 (segment (start 23.61 3.556) (end 23.61 11.306) (width 4.13) (layer F.Cu) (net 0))
 (segment (start 55.544376 11.424522) (end 51.274736 11.424522) (width 4.13) (layer F.Cu) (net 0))
 (segment (start 51.274736 11.424522) (end 47.356794 7.50658) (width 4.13) (layer F.Cu) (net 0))
 (segment (start 51.188851 3.674522) (end 55.544376 3.674522) (width 4.13) (layer F.Cu) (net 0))
 (segment (start 47.356794 7.50658) (end 51.188851 3.674522) (width 4.13) (layer F.Cu) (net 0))
 (segment (start 56.122 3.556) (end 60.39164 3.556) (width 4.13) (layer F.Cu) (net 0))
 (segment (start 64.309582 7.473942) (end 60.477525 11.306) (width 4.13) (layer F.Cu) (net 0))
 (segment (start 60.39164 3.556) (end 64.309582 7.473942) (width 4.13) (layer F.Cu) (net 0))
 (segment (start 60.477525 11.306) (end 56.122 11.306) (width 4.13) (layer F.Cu) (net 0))
 (segment (start 56.122 3.556) (end 56.122 11.306) (width 4.13) (layer F.Cu) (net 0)))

